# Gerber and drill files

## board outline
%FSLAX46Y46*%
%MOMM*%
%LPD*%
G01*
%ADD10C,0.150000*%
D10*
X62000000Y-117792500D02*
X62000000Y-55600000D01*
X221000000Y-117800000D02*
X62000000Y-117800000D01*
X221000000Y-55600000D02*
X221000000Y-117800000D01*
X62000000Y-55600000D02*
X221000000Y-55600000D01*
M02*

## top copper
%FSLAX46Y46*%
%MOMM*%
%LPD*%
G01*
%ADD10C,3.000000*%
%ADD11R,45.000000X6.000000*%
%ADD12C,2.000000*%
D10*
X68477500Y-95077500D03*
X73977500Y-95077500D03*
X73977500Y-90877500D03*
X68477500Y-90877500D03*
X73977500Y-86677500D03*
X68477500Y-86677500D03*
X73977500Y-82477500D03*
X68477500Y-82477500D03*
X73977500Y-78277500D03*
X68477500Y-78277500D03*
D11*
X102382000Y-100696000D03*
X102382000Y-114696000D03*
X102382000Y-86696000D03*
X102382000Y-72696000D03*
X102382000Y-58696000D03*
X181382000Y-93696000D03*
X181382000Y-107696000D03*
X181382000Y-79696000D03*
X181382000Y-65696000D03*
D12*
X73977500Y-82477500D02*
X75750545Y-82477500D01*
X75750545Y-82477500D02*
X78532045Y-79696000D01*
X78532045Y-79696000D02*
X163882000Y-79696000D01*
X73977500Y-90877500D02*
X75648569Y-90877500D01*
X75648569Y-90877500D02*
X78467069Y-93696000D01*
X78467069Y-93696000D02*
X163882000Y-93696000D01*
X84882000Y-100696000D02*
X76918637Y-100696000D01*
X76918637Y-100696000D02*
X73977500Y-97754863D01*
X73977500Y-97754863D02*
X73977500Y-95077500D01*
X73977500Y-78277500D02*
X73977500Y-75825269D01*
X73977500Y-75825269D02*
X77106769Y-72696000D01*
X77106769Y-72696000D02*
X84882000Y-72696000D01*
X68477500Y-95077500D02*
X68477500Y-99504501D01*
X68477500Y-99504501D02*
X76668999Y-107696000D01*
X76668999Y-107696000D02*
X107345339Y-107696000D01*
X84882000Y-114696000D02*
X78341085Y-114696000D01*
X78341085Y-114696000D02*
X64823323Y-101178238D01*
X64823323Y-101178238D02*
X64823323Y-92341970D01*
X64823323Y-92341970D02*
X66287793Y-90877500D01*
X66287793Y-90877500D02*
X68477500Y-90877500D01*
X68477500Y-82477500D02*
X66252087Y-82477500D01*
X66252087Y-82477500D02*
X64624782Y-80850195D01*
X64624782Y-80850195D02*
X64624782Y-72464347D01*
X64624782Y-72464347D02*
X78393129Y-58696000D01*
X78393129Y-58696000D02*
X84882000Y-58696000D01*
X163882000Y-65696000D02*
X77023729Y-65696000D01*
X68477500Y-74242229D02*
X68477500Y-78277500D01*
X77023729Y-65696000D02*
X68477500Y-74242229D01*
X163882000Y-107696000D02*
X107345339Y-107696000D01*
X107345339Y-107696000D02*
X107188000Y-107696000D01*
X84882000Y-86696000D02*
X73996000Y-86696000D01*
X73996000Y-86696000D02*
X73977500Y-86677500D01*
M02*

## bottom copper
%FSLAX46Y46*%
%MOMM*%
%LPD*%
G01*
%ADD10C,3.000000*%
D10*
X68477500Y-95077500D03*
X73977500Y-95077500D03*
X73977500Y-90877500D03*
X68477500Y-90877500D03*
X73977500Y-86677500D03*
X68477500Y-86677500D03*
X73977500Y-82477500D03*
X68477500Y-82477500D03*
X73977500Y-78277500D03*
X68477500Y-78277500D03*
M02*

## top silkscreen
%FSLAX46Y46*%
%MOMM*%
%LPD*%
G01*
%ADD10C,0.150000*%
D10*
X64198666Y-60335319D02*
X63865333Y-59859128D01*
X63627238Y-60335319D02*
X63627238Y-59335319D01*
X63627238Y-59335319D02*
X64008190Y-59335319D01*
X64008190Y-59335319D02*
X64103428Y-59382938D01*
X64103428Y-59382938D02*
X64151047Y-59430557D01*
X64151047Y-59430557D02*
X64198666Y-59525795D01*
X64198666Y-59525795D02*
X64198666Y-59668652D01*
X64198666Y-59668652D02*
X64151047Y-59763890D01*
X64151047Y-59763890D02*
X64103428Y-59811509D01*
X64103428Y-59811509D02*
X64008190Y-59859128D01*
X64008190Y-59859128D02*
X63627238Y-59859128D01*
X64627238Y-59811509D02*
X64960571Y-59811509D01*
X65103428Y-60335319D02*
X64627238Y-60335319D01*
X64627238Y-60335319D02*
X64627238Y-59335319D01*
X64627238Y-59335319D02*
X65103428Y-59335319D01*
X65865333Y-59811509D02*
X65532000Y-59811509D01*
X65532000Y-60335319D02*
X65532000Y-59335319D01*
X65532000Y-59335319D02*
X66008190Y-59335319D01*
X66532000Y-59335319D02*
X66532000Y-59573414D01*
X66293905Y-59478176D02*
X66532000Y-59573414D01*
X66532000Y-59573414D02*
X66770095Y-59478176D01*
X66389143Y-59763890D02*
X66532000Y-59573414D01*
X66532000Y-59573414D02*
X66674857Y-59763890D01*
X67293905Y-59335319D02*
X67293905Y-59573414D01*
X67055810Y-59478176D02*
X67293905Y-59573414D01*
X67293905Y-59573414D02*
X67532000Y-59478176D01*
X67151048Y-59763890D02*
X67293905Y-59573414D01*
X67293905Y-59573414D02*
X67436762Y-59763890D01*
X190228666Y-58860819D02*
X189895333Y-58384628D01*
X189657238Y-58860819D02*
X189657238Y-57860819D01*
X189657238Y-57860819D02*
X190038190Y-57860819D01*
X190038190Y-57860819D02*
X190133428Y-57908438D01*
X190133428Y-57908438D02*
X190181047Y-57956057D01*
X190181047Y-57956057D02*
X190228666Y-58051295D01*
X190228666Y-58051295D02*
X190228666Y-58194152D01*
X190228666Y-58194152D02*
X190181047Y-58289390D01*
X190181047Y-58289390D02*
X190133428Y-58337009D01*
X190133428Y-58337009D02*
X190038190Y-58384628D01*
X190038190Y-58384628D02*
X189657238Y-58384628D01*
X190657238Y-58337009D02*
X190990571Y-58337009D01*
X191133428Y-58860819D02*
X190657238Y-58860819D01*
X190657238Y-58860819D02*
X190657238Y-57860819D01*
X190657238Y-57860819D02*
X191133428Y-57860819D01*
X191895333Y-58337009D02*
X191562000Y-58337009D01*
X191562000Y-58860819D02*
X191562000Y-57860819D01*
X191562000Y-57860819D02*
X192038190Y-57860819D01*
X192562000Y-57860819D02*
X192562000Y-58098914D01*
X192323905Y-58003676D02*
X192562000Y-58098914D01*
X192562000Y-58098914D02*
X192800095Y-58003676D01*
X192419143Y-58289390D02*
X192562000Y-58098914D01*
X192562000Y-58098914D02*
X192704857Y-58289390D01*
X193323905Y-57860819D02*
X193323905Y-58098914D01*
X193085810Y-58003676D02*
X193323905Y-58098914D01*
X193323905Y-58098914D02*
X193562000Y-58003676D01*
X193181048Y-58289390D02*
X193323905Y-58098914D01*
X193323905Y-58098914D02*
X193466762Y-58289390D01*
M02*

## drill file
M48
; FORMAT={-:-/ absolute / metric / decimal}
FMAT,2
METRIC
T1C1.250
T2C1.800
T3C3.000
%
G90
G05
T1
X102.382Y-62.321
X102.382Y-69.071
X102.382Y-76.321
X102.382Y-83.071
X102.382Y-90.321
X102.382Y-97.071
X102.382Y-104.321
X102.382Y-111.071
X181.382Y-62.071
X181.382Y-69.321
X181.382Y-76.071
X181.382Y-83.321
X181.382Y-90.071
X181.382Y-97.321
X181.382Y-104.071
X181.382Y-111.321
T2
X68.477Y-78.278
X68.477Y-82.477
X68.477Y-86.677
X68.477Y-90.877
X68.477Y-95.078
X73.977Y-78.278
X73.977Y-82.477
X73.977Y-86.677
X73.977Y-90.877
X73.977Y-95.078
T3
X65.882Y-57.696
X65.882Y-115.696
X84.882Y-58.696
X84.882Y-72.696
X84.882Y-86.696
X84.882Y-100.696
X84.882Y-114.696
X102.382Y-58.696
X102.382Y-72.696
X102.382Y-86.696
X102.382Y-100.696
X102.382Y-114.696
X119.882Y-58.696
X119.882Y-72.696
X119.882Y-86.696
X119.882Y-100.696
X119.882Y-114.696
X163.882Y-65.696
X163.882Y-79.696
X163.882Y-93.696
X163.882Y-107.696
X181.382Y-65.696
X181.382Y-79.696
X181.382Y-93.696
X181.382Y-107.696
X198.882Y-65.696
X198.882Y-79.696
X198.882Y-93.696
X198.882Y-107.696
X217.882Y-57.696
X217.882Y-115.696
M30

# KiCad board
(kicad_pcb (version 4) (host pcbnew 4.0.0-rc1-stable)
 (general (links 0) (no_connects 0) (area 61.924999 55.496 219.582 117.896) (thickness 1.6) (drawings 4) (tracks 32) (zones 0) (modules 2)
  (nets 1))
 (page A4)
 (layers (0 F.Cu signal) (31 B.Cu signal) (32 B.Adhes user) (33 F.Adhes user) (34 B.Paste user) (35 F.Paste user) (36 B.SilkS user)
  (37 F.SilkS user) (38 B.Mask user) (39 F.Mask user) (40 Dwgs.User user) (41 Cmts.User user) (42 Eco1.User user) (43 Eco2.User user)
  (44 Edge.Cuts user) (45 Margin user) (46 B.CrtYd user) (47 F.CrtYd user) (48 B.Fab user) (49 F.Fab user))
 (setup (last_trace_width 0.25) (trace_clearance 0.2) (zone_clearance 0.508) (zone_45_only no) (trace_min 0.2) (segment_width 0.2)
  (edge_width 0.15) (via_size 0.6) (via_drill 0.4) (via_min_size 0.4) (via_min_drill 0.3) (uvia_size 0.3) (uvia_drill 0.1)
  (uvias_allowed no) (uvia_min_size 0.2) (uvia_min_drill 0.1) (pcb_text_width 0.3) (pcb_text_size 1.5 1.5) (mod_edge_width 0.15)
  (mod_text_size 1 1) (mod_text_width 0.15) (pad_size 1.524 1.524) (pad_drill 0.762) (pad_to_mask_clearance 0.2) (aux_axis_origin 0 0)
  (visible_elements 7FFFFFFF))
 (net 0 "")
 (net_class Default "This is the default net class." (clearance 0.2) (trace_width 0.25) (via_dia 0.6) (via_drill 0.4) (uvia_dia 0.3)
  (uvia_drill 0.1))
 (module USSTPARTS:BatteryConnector (layer F.Cu) (at 68.4775 95.0775)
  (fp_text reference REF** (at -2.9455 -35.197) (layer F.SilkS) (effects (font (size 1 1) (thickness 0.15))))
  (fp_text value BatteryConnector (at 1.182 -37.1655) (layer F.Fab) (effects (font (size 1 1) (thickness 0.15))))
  (pad "" np_thru_hole circle (at 0 0) (size 3 3) (drill 1.8) (layers *.Cu))
  (pad "" np_thru_hole circle (at 5.5 0) (size 3 3) (drill 1.8) (layers *.Cu))
  (pad "" np_thru_hole circle (at 5.5 -4.2) (size 3 3) (drill 1.8) (layers *.Cu))
  (pad "" np_thru_hole circle (at 0 -4.2) (size 3 3) (drill 1.8) (layers *.Cu))
  (pad "" np_thru_hole circle (at 5.5 -8.4) (size 3 3) (drill 1.8) (layers *.Cu))
  (pad "" np_thru_hole circle (at 0 -8.4) (size 3 3) (drill 1.8) (layers *.Cu))
  (pad "" np_thru_hole circle (at 5.5 -12.6) (size 3 3) (drill 1.8) (layers *.Cu))
  (pad "" np_thru_hole circle (at 0 -12.6) (size 3 3) (drill 1.8) (layers *.Cu))
  (pad "" np_thru_hole circle (at 5.5 -16.8) (size 3 3) (drill 1.8) (layers *.Cu))
  (pad "" np_thru_hole circle (at 0 -16.8) (size 3 3) (drill 1.8) (layers *.Cu)))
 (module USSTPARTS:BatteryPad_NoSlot (layer F.Cu) (at 102.382 100.696)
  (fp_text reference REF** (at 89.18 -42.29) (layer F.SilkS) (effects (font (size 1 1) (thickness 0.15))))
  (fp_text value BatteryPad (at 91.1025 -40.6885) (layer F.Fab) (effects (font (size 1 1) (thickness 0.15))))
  (pad 1 smd rect (at 0 0) (size 45 6) (layers F.Cu))
  (pad "" np_thru_hole circle (at 0 0) (size 3 3) (drill 3) (layers *.Cu))
  (pad "" np_thru_hole oval (at 0 -3.625) (size 1.25 1.25) (drill oval 1.25) (layers *.Cu))
  (pad "" np_thru_hole oval (at 0 3.625) (size 1.25 1.25) (drill oval 1.25) (layers *.Cu))
  (pad "" np_thru_hole circle (at 17.5 0) (size 3 3) (drill 3) (layers *.Cu))
  (pad "" np_thru_hole circle (at -17.5 0) (size 3 3) (drill 3) (layers *.Cu))
  (pad "" np_thru_hole circle (at 17.5 14) (size 3 3) (drill 3) (layers *.Cu))
  (pad "" np_thru_hole circle (at 0 14) (size 3 3) (drill 3) (layers *.Cu))
  (pad "" np_thru_hole oval (at 0 10.375) (size 1.25 1.25) (drill oval 1.25) (layers *.Cu))
  (pad "" np_thru_hole circle (at -36.5 15) (size 3 3) (drill 3) (layers *.Cu)) (pad 1 smd rect (at 0 14) (size 45 6) (layers F.Cu))
  (pad "" np_thru_hole circle (at 17.5 -14) (size 3 3) (drill 3) (layers *.Cu))
  (pad "" np_thru_hole oval (at 0 -10.375) (size 1.25 1.25) (drill oval 1.25) (layers *.Cu))
  (pad "" np_thru_hole circle (at 0 -14) (size 3 3) (drill 3) (layers *.Cu))
  (pad "" np_thru_hole oval (at 0 -17.625) (size 1.25 1.25) (drill oval 1.25) (layers *.Cu))
  (pad "" np_thru_hole circle (at -17.5 -14) (size 3 3) (drill 3) (layers *.Cu)) (pad 1 smd rect (at 0 -14) (size 45 6) (layers F.Cu))
  (pad "" np_thru_hole oval (at 0 -24.375) (size 1.25 1.25) (drill oval 1.25) (layers *.Cu))
  (pad "" np_thru_hole oval (at 0 -31.625) (size 1.25 1.25) (drill oval 1.25) (layers *.Cu))
  (pad "" np_thru_hole circle (at 17.5 -28) (size 3 3) (drill 3) (layers *.Cu))
  (pad "" np_thru_hole circle (at -17.5 -28) (size 3 3) (drill 3) (layers *.Cu))
  (pad "" np_thru_hole circle (at 0 -28) (size 3 3) (drill 3) (layers *.Cu)) (pad 1 smd rect (at 0 -28) (size 45 6) (layers F.Cu))
  (pad "" np_thru_hole circle (at -17.5 -42) (size 3 3) (drill 3) (layers *.Cu))
  (pad "" np_thru_hole circle (at 0 -42) (size 3 3) (drill 3) (layers *.Cu))
  (pad "" np_thru_hole circle (at 17.5 -42) (size 3 3) (drill 3) (layers *.Cu))
  (pad "" np_thru_hole oval (at 0 -38.375) (size 1.25 1.25) (drill oval 1.25) (layers *.Cu))
  (pad 1 smd rect (at 0 -42) (size 45 6) (layers F.Cu))
  (pad "" np_thru_hole oval (at 79 -24.625) (size 1.25 1.25) (drill oval 1.25) (layers *.Cu))
  (pad "" np_thru_hole circle (at 79 -7) (size 3 3) (drill 3) (layers *.Cu))
  (pad "" np_thru_hole oval (at 79 -10.625) (size 1.25 1.25) (drill oval 1.25) (layers *.Cu))
  (pad "" np_thru_hole circle (at 61.5 -7) (size 3 3) (drill 3) (layers *.Cu))
  (pad "" np_thru_hole oval (at 79 -3.375) (size 1.25 1.25) (drill oval 1.25) (layers *.Cu))
  (pad "" np_thru_hole oval (at 79 10.625) (size 1.25 1.25) (drill oval 1.25) (layers *.Cu))
  (pad "" np_thru_hole circle (at 96.5 7) (size 3 3) (drill 3) (layers *.Cu))
  (pad "" np_thru_hole circle (at 79 7) (size 3 3) (drill 3) (layers *.Cu))
  (pad "" np_thru_hole oval (at 79 3.375) (size 1.25 1.25) (drill oval 1.25) (layers *.Cu))
  (pad "" np_thru_hole circle (at 61.5 7) (size 3 3) (drill 3) (layers *.Cu))
  (pad "" np_thru_hole oval (at 79 -38.625) (size 1.25 1.25) (drill oval 1.25) (layers *.Cu))
  (pad "" np_thru_hole oval (at 79 -31.375) (size 1.25 1.25) (drill oval 1.25) (layers *.Cu))
  (pad "" np_thru_hole circle (at 96.5 -35) (size 3 3) (drill 3) (layers *.Cu))
  (pad "" np_thru_hole circle (at 61.5 -35) (size 3 3) (drill 3) (layers *.Cu))
  (pad "" np_thru_hole circle (at 79 -35) (size 3 3) (drill 3) (layers *.Cu))
  (pad "" np_thru_hole circle (at 96.5 -7) (size 3 3) (drill 3) (layers *.Cu))
  (pad "" np_thru_hole circle (at 96.5 -21) (size 3 3) (drill 3) (layers *.Cu))
  (pad "" np_thru_hole oval (at 79 -17.375) (size 1.25 1.25) (drill oval 1.25) (layers *.Cu))
  (pad "" np_thru_hole circle (at 79 -21) (size 3 3) (drill 3) (layers *.Cu))
  (pad "" np_thru_hole circle (at 61.5 -21) (size 3 3) (drill 3) (layers *.Cu)) (pad 1 smd rect (at 79 -7) (size 45 6) (layers F.Cu))
  (pad 1 smd rect (at 79 7) (size 45 6) (layers F.Cu)) (pad 1 smd rect (at 79 -21) (size 45 6) (layers F.Cu))
  (pad 1 smd rect (at 79 -35) (size 45 6) (layers F.Cu))
  (pad "" np_thru_hole circle (at -17.5 14) (size 3 3) (drill 3) (layers *.Cu))
  (pad "" np_thru_hole circle (at -36.5 -43) (size 3 3) (drill 3) (layers *.Cu))
  (pad "" np_thru_hole circle (at 115.5 15) (size 3 3) (drill 3) (layers *.Cu))
  (pad "" np_thru_hole circle (at 115.5 -43) (size 3 3) (drill 3) (layers *.Cu)))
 (gr_line (start 62 117.7925) (end 62 55.6) (layer Edge.Cuts) (width 0.15))
 (gr_line (start 221 117.8) (end 62 117.8) (layer Edge.Cuts) (width 0.15))
 (gr_line (start 221 55.6) (end 221 117.8) (layer Edge.Cuts) (width 0.15))
 (gr_line (start 62 55.6) (end 221 55.6) (layer Edge.Cuts) (width 0.15))
 (segment (start 73.9775 82.4775) (end 75.750545 82.4775) (width 2) (layer F.Cu) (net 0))
 (segment (start 75.750545 82.4775) (end 78.532045 79.696) (width 2) (layer F.Cu) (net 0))
 (segment (start 78.532045 79.696) (end 163.882 79.696) (width 2) (layer F.Cu) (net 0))
 (segment (start 73.9775 90.8775) (end 75.648569 90.8775) (width 2) (layer F.Cu) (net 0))
 (segment (start 75.648569 90.8775) (end 78.467069 93.696) (width 2) (layer F.Cu) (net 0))
 (segment (start 78.467069 93.696) (end 163.882 93.696) (width 2) (layer F.Cu) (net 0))
 (segment (start 84.882 100.696) (end 76.918637 100.696) (width 2) (layer F.Cu) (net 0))
 (segment (start 76.918637 100.696) (end 73.9775 97.754863) (width 2) (layer F.Cu) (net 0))
 (segment (start 73.9775 97.754863) (end 73.9775 95.0775) (width 2) (layer F.Cu) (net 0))
 (segment (start 73.9775 78.2775) (end 73.9775 75.825269) (width 2) (layer F.Cu) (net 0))
 (segment (start 73.9775 75.825269) (end 77.106769 72.696) (width 2) (layer F.Cu) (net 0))
 (segment (start 77.106769 72.696) (end 84.882 72.696) (width 2) (layer F.Cu) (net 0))
 (segment (start 68.4775 95.0775) (end 68.4775 99.504501) (width 2) (layer F.Cu) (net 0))
 (segment (start 68.4775 99.504501) (end 76.668999 107.696) (width 2) (layer F.Cu) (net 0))
 (segment (start 76.668999 107.696) (end 107.345339 107.696) (width 2) (layer F.Cu) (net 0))
 (segment (start 84.882 114.696) (end 78.341085 114.696) (width 2) (layer F.Cu) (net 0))
 (segment (start 78.341085 114.696) (end 64.823323 101.178238) (width 2) (layer F.Cu) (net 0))
 (segment (start 64.823323 101.178238) (end 64.823323 92.34197) (width 2) (layer F.Cu) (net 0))
 (segment (start 64.823323 92.34197) (end 66.287793 90.8775) (width 2) (layer F.Cu) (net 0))
 (segment (start 66.287793 90.8775) (end 68.4775 90.8775) (width 2) (layer F.Cu) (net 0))
 (segment (start 68.4775 82.4775) (end 66.252087 82.4775) (width 2) (layer F.Cu) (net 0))
 (segment (start 66.252087 82.4775) (end 64.624782 80.850195) (width 2) (layer F.Cu) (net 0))
 (segment (start 64.624782 80.850195) (end 64.624782 72.464347) (width 2) (layer F.Cu) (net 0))
 (segment (start 64.624782 72.464347) (end 78.393129 58.696) (width 2) (layer F.Cu) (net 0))
 (segment (start 78.393129 58.696) (end 84.882 58.696) (width 2) (layer F.Cu) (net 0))
 (segment (start 163.882 65.696) (end 77.023729 65.696) (width 2) (layer F.Cu) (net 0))
 (segment (start 68.4775 74.242229) (end 68.4775 78.2775) (width 2) (layer F.Cu) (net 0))
 (segment (start 77.023729 65.696) (end 68.4775 74.242229) (width 2) (layer F.Cu) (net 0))
 (segment (start 163.882 107.696) (end 107.345339 107.696) (width 2) (layer F.Cu) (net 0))
 (segment (start 107.345339 107.696) (end 107.188 107.696) (width 2) (layer F.Cu) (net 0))
 (segment (start 84.882 86.696) (end 73.996 86.696) (width 2) (layer F.Cu) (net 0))
 (segment (start 73.996 86.696) (end 73.9775 86.6775) (width 2) (layer F.Cu) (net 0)))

